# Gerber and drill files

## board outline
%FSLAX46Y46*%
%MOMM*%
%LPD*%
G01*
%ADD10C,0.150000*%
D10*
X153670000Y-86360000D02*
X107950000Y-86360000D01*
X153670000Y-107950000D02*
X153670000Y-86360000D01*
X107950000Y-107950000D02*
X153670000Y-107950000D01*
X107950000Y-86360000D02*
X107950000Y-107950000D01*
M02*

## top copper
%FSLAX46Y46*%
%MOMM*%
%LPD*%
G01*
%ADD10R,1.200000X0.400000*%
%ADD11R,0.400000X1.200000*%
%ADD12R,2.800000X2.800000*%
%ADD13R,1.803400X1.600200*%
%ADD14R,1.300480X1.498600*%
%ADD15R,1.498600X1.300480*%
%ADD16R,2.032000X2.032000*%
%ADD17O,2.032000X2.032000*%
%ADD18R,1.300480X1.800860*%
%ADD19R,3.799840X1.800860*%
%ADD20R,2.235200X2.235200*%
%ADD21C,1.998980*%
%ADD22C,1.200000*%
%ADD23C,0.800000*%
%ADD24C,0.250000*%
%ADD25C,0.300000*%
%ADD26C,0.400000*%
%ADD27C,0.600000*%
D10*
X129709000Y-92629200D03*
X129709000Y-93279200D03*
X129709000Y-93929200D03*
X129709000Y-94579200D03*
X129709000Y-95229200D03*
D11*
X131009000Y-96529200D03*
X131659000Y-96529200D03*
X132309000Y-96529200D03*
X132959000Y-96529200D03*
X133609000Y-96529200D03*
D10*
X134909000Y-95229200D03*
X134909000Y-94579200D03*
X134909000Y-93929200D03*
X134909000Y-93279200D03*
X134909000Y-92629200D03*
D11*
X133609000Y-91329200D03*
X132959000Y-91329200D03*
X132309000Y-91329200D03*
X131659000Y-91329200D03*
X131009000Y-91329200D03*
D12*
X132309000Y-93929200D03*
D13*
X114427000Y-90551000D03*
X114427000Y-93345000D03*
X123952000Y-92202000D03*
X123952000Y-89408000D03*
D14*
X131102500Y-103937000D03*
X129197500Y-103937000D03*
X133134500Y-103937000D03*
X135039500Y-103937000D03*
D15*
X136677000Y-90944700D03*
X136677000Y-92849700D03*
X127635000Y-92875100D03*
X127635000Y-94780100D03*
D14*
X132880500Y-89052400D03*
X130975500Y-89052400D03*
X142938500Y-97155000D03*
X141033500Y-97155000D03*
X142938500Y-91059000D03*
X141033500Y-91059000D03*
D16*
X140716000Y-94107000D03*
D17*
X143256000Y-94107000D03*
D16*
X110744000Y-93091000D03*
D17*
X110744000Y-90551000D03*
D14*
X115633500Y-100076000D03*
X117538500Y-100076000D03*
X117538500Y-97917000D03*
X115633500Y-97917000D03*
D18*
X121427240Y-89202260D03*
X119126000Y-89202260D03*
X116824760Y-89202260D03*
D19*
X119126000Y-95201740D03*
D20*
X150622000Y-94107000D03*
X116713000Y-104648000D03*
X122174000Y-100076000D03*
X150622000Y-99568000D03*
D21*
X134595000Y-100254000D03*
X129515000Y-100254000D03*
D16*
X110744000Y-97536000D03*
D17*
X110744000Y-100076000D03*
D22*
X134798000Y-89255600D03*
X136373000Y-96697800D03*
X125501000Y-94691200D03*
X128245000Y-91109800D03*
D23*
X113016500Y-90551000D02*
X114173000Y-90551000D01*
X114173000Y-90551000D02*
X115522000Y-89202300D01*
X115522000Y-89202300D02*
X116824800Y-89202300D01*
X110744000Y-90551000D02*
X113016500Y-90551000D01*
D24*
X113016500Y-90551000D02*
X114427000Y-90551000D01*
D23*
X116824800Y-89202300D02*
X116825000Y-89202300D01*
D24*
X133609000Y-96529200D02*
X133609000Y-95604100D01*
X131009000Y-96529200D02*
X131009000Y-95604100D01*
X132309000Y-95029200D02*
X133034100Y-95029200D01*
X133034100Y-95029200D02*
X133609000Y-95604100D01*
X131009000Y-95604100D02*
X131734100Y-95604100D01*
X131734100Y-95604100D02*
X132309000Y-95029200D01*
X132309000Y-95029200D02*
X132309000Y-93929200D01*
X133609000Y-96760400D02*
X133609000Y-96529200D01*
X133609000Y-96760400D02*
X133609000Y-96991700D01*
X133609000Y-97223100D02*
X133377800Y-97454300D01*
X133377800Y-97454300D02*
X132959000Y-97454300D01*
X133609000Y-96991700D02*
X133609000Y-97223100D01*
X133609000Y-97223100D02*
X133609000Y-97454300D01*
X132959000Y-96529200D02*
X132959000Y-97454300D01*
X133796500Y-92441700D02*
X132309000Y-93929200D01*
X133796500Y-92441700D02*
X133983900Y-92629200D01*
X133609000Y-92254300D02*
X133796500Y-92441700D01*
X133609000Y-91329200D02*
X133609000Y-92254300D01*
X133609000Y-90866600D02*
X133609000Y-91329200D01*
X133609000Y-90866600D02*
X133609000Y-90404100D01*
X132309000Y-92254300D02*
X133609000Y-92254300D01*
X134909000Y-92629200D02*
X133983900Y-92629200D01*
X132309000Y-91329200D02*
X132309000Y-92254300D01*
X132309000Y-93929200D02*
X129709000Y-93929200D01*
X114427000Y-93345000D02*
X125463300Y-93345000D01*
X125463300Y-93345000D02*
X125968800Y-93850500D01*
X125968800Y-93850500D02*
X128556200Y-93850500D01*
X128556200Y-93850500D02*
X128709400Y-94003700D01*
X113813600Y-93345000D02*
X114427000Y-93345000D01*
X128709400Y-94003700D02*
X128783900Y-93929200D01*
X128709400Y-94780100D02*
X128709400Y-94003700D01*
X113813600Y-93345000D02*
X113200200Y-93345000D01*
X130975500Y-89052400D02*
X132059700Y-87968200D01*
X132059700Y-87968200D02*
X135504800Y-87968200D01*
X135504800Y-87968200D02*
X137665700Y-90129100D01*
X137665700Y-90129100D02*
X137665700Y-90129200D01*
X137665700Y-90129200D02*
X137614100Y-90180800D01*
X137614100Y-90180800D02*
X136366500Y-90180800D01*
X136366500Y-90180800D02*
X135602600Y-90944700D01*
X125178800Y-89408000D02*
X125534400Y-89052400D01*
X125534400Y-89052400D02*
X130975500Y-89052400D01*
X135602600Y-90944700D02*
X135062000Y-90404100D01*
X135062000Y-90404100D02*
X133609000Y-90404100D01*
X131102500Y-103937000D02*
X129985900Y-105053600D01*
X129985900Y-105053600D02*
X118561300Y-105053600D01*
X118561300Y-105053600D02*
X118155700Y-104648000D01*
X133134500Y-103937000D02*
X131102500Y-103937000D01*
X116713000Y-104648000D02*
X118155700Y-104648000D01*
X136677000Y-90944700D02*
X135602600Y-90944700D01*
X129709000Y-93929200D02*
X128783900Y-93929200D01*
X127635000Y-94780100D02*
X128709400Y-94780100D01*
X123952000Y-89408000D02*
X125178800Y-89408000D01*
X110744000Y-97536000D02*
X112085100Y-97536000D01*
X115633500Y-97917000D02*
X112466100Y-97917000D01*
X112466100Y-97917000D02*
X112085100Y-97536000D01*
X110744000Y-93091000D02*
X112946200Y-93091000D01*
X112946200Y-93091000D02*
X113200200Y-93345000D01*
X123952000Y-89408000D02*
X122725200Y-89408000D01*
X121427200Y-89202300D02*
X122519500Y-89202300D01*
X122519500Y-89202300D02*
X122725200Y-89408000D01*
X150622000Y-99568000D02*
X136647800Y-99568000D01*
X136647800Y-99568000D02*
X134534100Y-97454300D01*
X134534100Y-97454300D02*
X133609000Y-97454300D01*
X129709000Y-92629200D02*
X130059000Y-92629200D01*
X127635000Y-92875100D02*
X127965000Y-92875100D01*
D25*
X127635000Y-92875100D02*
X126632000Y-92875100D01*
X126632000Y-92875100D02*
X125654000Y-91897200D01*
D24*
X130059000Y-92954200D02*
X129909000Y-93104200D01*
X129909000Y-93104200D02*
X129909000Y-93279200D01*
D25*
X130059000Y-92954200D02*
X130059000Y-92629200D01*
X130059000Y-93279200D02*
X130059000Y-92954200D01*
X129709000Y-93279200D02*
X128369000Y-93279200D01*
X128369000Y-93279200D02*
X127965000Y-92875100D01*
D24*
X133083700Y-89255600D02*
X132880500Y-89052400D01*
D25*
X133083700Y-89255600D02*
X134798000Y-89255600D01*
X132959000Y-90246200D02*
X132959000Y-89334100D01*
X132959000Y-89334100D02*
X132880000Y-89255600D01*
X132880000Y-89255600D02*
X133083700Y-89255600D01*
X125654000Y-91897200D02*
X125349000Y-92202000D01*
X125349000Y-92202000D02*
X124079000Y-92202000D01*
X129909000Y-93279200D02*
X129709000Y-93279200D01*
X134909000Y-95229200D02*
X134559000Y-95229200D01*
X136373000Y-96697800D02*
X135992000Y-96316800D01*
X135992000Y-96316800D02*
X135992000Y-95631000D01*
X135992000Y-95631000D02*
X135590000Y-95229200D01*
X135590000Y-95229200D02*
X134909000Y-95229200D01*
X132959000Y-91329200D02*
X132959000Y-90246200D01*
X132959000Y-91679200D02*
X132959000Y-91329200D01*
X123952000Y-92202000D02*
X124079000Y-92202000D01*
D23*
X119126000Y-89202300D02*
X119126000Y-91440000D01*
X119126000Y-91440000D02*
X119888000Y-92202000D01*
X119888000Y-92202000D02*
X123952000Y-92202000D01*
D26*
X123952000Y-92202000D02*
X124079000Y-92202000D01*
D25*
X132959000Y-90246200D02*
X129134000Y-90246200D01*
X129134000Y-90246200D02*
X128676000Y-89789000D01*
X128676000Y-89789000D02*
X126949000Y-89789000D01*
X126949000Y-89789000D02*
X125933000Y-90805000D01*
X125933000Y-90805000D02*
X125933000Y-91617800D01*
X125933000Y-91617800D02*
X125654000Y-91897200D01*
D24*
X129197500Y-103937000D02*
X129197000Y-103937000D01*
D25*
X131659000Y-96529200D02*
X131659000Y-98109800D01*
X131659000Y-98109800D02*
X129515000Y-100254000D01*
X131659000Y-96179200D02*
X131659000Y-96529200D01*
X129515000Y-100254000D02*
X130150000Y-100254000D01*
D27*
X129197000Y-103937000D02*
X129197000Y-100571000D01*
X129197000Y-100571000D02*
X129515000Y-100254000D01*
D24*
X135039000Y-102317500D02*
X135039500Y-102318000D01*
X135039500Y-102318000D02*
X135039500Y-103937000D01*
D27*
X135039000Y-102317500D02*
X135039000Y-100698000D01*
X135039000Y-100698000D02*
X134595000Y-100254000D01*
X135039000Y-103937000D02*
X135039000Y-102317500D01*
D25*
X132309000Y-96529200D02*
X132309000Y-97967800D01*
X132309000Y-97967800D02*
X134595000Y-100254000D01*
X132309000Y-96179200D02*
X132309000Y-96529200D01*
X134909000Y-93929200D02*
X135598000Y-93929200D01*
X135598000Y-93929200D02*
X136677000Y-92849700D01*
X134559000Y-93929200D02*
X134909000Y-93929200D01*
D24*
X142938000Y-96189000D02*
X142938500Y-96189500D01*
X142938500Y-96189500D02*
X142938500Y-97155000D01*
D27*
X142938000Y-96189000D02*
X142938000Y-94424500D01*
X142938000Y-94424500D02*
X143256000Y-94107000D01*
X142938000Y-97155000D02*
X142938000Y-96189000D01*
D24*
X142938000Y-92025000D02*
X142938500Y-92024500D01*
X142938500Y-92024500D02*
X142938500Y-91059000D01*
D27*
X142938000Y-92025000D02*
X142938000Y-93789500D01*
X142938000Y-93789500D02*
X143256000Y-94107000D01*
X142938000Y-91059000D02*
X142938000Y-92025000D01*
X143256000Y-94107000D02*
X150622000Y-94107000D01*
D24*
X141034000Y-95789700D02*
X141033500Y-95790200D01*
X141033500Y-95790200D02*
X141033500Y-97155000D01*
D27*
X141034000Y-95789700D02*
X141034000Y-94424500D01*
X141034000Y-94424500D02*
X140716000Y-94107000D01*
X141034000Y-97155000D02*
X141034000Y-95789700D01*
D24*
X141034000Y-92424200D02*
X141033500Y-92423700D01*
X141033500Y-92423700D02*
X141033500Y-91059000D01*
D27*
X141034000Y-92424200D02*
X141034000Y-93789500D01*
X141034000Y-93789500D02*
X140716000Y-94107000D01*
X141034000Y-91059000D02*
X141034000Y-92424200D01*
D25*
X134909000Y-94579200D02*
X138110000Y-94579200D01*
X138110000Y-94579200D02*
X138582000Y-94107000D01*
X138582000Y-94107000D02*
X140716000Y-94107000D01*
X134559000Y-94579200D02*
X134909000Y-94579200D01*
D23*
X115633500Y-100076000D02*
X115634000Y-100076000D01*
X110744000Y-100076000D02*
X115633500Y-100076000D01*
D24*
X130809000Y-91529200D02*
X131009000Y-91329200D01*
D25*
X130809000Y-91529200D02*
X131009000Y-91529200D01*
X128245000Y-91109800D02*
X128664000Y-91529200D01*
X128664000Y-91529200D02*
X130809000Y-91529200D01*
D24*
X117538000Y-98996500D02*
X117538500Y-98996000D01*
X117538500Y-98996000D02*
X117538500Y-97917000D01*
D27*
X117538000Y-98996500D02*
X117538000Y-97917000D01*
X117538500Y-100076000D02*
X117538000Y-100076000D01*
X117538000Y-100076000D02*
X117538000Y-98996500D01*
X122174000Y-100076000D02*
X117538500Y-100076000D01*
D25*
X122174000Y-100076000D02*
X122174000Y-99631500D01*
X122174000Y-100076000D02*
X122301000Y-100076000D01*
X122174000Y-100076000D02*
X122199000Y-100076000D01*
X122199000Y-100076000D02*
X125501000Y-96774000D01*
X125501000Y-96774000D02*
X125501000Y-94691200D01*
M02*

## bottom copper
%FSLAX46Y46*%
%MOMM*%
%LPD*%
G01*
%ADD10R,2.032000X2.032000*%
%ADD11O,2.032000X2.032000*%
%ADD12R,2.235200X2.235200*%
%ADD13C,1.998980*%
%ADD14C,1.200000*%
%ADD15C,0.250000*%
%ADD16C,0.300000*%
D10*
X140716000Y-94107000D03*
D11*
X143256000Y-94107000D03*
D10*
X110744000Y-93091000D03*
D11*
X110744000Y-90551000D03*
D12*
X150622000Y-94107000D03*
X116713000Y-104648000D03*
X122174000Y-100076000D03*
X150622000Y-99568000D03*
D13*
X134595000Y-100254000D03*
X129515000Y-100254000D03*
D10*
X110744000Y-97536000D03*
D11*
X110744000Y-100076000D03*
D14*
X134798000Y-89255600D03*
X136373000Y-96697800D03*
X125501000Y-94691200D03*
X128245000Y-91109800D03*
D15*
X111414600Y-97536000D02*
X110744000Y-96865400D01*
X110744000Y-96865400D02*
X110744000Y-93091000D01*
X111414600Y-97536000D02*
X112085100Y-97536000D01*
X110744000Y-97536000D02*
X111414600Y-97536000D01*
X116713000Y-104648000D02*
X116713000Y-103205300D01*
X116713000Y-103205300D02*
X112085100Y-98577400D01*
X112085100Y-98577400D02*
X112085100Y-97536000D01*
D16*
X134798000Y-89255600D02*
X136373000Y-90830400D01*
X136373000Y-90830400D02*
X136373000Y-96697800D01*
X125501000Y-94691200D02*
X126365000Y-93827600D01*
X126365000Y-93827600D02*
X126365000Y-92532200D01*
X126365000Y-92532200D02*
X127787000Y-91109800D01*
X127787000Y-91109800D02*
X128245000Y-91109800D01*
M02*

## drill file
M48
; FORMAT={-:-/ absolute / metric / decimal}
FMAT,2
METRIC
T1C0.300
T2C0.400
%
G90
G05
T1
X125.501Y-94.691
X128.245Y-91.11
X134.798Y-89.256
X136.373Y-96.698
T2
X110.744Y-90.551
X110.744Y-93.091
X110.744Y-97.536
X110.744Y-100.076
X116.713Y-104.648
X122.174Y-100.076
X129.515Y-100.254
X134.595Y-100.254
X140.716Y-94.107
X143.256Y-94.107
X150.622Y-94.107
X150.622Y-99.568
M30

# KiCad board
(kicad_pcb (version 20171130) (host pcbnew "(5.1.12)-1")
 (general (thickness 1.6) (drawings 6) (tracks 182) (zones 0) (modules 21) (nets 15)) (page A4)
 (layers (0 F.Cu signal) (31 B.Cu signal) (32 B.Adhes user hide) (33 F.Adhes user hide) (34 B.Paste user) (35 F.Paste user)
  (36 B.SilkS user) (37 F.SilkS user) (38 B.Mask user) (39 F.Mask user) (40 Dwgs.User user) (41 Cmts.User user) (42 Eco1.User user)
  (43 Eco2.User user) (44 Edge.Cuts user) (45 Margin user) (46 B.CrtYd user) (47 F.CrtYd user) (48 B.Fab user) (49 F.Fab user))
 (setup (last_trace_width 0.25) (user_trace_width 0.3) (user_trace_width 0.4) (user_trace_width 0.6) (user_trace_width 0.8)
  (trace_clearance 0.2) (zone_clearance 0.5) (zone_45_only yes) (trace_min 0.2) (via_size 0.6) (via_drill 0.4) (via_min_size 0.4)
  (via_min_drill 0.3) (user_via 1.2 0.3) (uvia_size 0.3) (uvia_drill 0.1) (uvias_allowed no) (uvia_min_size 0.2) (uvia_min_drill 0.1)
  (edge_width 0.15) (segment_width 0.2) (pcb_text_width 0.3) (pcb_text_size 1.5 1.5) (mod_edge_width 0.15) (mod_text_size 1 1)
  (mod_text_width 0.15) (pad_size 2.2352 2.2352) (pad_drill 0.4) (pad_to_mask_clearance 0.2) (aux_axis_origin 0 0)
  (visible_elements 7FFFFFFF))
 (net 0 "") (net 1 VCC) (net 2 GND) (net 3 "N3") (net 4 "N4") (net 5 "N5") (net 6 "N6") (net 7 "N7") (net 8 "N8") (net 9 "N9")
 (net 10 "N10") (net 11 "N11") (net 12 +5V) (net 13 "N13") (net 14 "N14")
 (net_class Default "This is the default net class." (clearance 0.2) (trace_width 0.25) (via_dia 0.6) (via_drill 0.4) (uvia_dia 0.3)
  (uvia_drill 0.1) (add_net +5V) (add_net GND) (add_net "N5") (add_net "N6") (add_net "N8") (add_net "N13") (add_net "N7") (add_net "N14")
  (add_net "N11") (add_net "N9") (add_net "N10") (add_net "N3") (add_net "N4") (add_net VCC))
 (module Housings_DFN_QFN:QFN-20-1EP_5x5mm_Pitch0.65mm (layer F.Cu) (at 132.309 93.9292)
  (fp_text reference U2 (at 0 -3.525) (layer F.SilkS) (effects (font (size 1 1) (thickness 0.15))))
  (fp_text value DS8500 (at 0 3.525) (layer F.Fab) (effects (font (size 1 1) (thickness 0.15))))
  (pad 1 smd rect (at -2.6 -1.3) (size 1.2 0.4) (layers F.Cu F.Paste F.Mask) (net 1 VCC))
  (pad 2 smd rect (at -2.6 -0.65) (size 1.2 0.4) (layers F.Cu F.Paste F.Mask) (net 1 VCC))
  (pad 3 smd rect (at -2.6 0) (size 1.2 0.4) (layers F.Cu F.Paste F.Mask) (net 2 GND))
  (pad 4 smd rect (at -2.6 0.65) (size 1.2 0.4) (layers F.Cu F.Paste F.Mask) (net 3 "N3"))
  (pad 5 smd rect (at -2.6 1.3) (size 1.2 0.4) (layers F.Cu F.Paste F.Mask) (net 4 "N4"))
  (pad 6 smd rect (at -1.3 2.6 90) (size 1.2 0.4) (layers F.Cu F.Paste F.Mask) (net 2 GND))
  (pad 7 smd rect (at -0.65 2.6 90) (size 1.2 0.4) (layers F.Cu F.Paste F.Mask) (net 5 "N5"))
  (pad 8 smd rect (at 0 2.6 90) (size 1.2 0.4) (layers F.Cu F.Paste F.Mask) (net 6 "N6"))
  (pad 9 smd rect (at 0.65 2.6 90) (size 1.2 0.4) (layers F.Cu F.Paste F.Mask) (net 2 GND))
  (pad 10 smd rect (at 1.3 2.6 90) (size 1.2 0.4) (layers F.Cu F.Paste F.Mask) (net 2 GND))
  (pad 11 smd rect (at 2.6 1.3) (size 1.2 0.4) (layers F.Cu F.Paste F.Mask) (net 1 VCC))
  (pad 12 smd rect (at 2.6 0.65) (size 1.2 0.4) (layers F.Cu F.Paste F.Mask) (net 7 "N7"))
  (pad 13 smd rect (at 2.6 0) (size 1.2 0.4) (layers F.Cu F.Paste F.Mask) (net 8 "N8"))
  (pad 14 smd rect (at 2.6 -0.65) (size 1.2 0.4) (layers F.Cu F.Paste F.Mask) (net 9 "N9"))
  (pad 15 smd rect (at 2.6 -1.3) (size 1.2 0.4) (layers F.Cu F.Paste F.Mask) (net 2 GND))
  (pad 16 smd rect (at 1.3 -2.6 90) (size 1.2 0.4) (layers F.Cu F.Paste F.Mask) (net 2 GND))
  (pad 17 smd rect (at 0.65 -2.6 90) (size 1.2 0.4) (layers F.Cu F.Paste F.Mask) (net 1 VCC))
  (pad 18 smd rect (at 0 -2.6 90) (size 1.2 0.4) (layers F.Cu F.Paste F.Mask) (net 2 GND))
  (pad 19 smd rect (at -0.65 -2.6 90) (size 1.2 0.4) (layers F.Cu F.Paste F.Mask) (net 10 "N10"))
  (pad 20 smd rect (at -1.3 -2.6 90) (size 1.2 0.4) (layers F.Cu F.Paste F.Mask) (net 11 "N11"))
  (pad 21 smd rect (at 0 0) (size 2.8 2.8) (layers F.Cu F.Paste F.Mask) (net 2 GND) (solder_paste_margin_ratio -0.2)))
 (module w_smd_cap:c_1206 (layer F.Cu) (at 114.427 91.948 90)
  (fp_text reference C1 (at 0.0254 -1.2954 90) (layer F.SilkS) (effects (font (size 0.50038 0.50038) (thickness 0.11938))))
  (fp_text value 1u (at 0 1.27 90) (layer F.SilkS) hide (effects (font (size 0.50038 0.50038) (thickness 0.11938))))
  (pad 1 smd rect (at 1.397 0 90) (size 1.6002 1.8034) (layers F.Cu F.Paste F.Mask) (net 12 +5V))
  (pad 2 smd rect (at -1.397 0 90) (size 1.6002 1.8034) (layers F.Cu F.Paste F.Mask) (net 2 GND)))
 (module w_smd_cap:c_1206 (layer F.Cu) (at 123.952 90.805 270)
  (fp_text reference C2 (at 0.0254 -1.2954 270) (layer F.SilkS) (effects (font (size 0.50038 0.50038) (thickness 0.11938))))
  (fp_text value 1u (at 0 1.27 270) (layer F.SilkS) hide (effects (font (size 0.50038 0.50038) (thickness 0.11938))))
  (pad 1 smd rect (at 1.397 0 270) (size 1.6002 1.8034) (layers F.Cu F.Paste F.Mask) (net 1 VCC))
  (pad 2 smd rect (at -1.397 0 270) (size 1.6002 1.8034) (layers F.Cu F.Paste F.Mask) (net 2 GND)))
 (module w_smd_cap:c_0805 (layer F.Cu) (at 130.15 103.937)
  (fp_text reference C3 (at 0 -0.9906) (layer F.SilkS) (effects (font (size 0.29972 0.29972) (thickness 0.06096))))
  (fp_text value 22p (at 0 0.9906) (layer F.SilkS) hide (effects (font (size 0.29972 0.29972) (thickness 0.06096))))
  (pad 1 smd rect (at 0.9525 0) (size 1.30048 1.4986) (layers F.Cu F.Paste F.Mask) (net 2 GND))
  (pad 2 smd rect (at -0.9525 0) (size 1.30048 1.4986) (layers F.Cu F.Paste F.Mask) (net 5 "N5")))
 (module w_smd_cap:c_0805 (layer F.Cu) (at 134.087 103.937 180)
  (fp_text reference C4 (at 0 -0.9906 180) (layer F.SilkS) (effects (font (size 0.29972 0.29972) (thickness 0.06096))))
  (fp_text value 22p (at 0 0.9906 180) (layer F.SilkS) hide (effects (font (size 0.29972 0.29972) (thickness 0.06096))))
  (pad 1 smd rect (at 0.9525 0 180) (size 1.30048 1.4986) (layers F.Cu F.Paste F.Mask) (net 2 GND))
  (pad 2 smd rect (at -0.9525 0 180) (size 1.30048 1.4986) (layers F.Cu F.Paste F.Mask) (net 6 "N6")))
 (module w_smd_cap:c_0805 (layer F.Cu) (at 136.677 91.8972 90)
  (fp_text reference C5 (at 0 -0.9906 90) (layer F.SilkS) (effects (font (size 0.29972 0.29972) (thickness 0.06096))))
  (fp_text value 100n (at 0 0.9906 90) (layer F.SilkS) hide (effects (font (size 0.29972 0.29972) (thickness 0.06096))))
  (pad 1 smd rect (at 0.9525 0 90) (size 1.30048 1.4986) (layers F.Cu F.Paste F.Mask) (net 2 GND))
  (pad 2 smd rect (at -0.9525 0 90) (size 1.30048 1.4986) (layers F.Cu F.Paste F.Mask) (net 8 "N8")))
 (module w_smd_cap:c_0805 (layer F.Cu) (at 127.635 93.8276 90)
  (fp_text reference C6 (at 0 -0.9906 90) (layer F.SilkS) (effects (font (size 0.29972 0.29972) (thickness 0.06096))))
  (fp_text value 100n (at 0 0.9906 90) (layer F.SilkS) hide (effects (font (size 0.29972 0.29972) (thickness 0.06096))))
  (pad 1 smd rect (at 0.9525 0 90) (size 1.30048 1.4986) (layers F.Cu F.Paste F.Mask) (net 1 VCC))
  (pad 2 smd rect (at -0.9525 0 90) (size 1.30048 1.4986) (layers F.Cu F.Paste F.Mask) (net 2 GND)))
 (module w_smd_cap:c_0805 (layer F.Cu) (at 131.928 89.0524)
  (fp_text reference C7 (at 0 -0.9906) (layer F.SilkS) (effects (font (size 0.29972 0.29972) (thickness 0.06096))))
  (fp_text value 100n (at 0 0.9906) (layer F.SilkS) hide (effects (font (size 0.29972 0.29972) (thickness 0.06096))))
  (pad 1 smd rect (at 0.9525 0) (size 1.30048 1.4986) (layers F.Cu F.Paste F.Mask) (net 1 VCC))
  (pad 2 smd rect (at -0.9525 0) (size 1.30048 1.4986) (layers F.Cu F.Paste F.Mask) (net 2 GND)))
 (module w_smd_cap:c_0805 (layer F.Cu) (at 141.986 97.155)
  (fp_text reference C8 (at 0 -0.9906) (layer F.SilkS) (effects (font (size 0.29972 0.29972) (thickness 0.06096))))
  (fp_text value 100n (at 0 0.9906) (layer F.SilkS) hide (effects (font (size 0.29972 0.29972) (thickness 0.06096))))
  (pad 1 smd rect (at 0.9525 0) (size 1.30048 1.4986) (layers F.Cu F.Paste F.Mask) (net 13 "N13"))
  (pad 2 smd rect (at -0.9525 0) (size 1.30048 1.4986) (layers F.Cu F.Paste F.Mask) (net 7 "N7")))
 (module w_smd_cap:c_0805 (layer F.Cu) (at 141.986 91.059)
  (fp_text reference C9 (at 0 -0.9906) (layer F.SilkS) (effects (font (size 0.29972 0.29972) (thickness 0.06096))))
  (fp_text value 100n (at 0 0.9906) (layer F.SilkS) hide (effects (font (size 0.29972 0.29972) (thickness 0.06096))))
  (pad 1 smd rect (at 0.9525 0) (size 1.30048 1.4986) (layers F.Cu F.Paste F.Mask) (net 13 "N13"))
  (pad 2 smd rect (at -0.9525 0) (size 1.30048 1.4986) (layers F.Cu F.Paste F.Mask) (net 7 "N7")))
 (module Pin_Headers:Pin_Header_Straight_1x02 (layer F.Cu) (at 140.716 94.107 90)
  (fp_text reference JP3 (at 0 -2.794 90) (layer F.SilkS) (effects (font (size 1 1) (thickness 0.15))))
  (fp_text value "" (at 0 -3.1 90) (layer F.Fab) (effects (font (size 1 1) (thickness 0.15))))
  (pad 1 thru_hole rect (at 0 0 90) (size 2.032 2.032) (drill 0.4) (layers *.Cu *.Mask F.SilkS) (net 7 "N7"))
  (pad 2 thru_hole oval (at 0 2.54 90) (size 2.032 2.032) (drill 0.4) (layers *.Cu *.Mask F.SilkS) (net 13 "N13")))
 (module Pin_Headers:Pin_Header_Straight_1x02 (layer F.Cu) (at 110.744 93.091 180)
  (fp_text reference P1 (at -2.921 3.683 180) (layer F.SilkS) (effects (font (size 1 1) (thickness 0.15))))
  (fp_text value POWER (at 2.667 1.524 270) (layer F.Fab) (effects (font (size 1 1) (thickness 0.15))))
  (pad 1 thru_hole rect (at 0 0 180) (size 2.032 2.032) (drill 0.4) (layers *.Cu *.Mask F.SilkS) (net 2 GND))
  (pad 2 thru_hole oval (at 0 2.54 180) (size 2.032 2.032) (drill 0.4) (layers *.Cu *.Mask F.SilkS) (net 12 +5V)))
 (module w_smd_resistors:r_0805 (layer F.Cu) (at 116.586 100.076 180)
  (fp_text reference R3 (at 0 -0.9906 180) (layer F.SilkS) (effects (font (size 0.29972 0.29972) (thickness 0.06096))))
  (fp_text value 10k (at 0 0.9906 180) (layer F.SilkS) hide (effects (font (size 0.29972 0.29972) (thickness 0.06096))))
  (pad 1 smd rect (at 0.9525 0 180) (size 1.30048 1.4986) (layers F.Cu F.Paste F.Mask) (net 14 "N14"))
  (pad 2 smd rect (at -0.9525 0 180) (size 1.30048 1.4986) (layers F.Cu F.Paste F.Mask) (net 11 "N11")))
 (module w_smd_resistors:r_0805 (layer F.Cu) (at 116.586 97.917)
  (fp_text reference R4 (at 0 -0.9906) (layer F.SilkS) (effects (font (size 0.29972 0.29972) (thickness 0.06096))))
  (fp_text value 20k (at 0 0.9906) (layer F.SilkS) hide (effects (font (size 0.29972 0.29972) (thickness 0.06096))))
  (pad 1 smd rect (at 0.9525 0) (size 1.30048 1.4986) (layers F.Cu F.Paste F.Mask) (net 11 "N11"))
  (pad 2 smd rect (at -0.9525 0) (size 1.30048 1.4986) (layers F.Cu F.Paste F.Mask) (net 2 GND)))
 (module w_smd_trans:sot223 (layer F.Cu) (at 119.126 92.202 180)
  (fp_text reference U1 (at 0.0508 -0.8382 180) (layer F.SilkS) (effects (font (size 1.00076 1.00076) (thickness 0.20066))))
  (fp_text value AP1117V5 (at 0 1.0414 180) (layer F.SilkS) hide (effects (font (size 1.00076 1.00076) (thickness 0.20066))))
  (pad 1 smd rect (at -2.30124 2.99974 180) (size 1.30048 1.80086) (layers F.Cu F.Paste F.Mask) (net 2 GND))
  (pad 2 smd rect (at 0 2.99974 180) (size 1.30048 1.80086) (layers F.Cu F.Paste F.Mask) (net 1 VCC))
  (pad 3 smd rect (at 2.30124 2.99974 180) (size 1.30048 1.80086) (layers F.Cu F.Paste F.Mask) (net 12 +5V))
  (pad 4 smd rect (at 0 -2.99974 180) (size 3.79984 1.80086) (layers F.Cu F.Paste F.Mask)))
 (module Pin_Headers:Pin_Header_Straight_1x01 (layer F.Cu) (at 150.622 94.107)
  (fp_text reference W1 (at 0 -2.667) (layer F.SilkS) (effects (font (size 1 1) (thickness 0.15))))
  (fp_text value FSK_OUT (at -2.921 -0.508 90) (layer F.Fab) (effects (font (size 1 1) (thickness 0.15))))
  (pad 1 thru_hole rect (at 0 0) (size 2.2352 2.2352) (drill 0.4) (layers *.Cu *.Mask F.SilkS) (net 13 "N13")))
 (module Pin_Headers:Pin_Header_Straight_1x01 (layer F.Cu) (at 116.713 104.648)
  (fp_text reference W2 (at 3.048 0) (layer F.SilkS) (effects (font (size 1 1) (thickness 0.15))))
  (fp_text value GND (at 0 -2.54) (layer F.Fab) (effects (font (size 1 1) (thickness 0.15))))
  (pad 1 thru_hole rect (at 0 0) (size 2.2352 2.2352) (drill 0.4) (layers *.Cu *.Mask F.SilkS) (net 2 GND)))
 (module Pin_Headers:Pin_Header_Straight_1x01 (layer F.Cu) (at 122.174 100.076)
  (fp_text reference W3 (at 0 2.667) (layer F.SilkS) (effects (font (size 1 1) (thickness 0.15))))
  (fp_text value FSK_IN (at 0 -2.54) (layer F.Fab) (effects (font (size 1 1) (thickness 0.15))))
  (pad 1 thru_hole rect (at 0 0) (size 2.2352 2.2352) (drill 0.4) (layers *.Cu *.Mask F.SilkS) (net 11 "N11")))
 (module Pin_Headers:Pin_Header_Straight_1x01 (layer F.Cu) (at 150.622 99.568)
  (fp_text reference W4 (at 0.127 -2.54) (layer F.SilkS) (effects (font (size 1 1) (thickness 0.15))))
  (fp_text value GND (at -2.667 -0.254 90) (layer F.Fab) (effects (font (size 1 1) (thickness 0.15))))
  (pad 1 thru_hole rect (at 0 0) (size 2.2352 2.2352) (drill 0.4) (layers *.Cu *.Mask F.SilkS) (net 2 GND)))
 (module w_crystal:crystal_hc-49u (layer F.Cu) (at 132.055 100.254 180) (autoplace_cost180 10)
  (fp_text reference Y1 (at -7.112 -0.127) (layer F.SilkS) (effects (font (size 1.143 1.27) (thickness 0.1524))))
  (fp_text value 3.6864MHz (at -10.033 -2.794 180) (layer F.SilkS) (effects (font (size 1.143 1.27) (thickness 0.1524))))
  (pad 1 thru_hole circle (at -2.54 0 180) (size 1.99898 1.99898) (drill 0.4) (layers *.Cu *.Mask F.SilkS) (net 6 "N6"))
  (pad 2 thru_hole circle (at 2.54 0 180) (size 1.99898 1.99898) (drill 0.4) (layers *.Cu *.Mask F.SilkS) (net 5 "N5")))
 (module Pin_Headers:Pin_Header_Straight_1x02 (layer F.Cu) (at 110.744 97.536)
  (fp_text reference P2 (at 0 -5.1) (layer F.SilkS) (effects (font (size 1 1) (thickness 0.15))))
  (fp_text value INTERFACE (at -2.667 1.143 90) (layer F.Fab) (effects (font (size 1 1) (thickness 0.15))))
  (pad 1 thru_hole rect (at 0 0) (size 2.032 2.032) (drill 0.4) (layers *.Cu *.Mask F.SilkS) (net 2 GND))
  (pad 2 thru_hole oval (at 0 2.54) (size 2.032 2.032) (drill 0.4) (layers *.Cu *.Mask F.SilkS) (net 14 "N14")))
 (gr_line (start 153.67 86.36) (end 107.95 86.36) (angle 90) (layer Edge.Cuts) (width 0.15))
 (gr_line (start 153.67 107.95) (end 153.67 86.36) (angle 90) (layer Edge.Cuts) (width 0.15))
 (gr_line (start 107.95 107.95) (end 153.67 107.95) (angle 90) (layer Edge.Cuts) (width 0.15))
 (gr_line (start 107.95 86.36) (end 107.95 107.95) (angle 90) (layer Edge.Cuts) (width 0.15))
 (segment (start 113.0165 90.551) (end 114.173 90.551) (width 0.8) (layer F.Cu) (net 12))
 (segment (start 114.173 90.551) (end 115.522 89.2023) (width 0.8) (layer F.Cu) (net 12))
 (segment (start 115.522 89.2023) (end 116.8248 89.2023) (width 0.8) (layer F.Cu) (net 12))
 (segment (start 110.744 90.551) (end 113.0165 90.551) (width 0.8) (layer F.Cu) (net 12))
 (segment (start 113.0165 90.551) (end 114.427 90.551) (width 0.25) (layer F.Cu) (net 12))
 (segment (start 116.8248 89.2023) (end 116.825 89.2023) (width 0.8) (layer F.Cu) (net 12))
 (segment (start 133.609 96.5292) (end 133.609 95.6041) (width 0.25) (layer F.Cu) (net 2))
 (segment (start 131.009 96.5292) (end 131.009 95.6041) (width 0.25) (layer F.Cu) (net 2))
 (segment (start 132.309 95.0292) (end 133.0341 95.0292) (width 0.25) (layer F.Cu) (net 2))
 (segment (start 133.0341 95.0292) (end 133.609 95.6041) (width 0.25) (layer F.Cu) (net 2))
 (segment (start 131.009 95.6041) (end 131.7341 95.6041) (width 0.25) (layer F.Cu) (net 2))
 (segment (start 131.7341 95.6041) (end 132.309 95.0292) (width 0.25) (layer F.Cu) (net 2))
 (segment (start 132.309 95.0292) (end 132.309 93.9292) (width 0.25) (layer F.Cu) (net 2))
 (segment (start 133.609 96.7604) (end 133.609 96.5292) (width 0.25) (layer F.Cu) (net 2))
 (segment (start 133.609 96.7604) (end 133.609 96.9917) (width 0.25) (layer F.Cu) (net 2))
 (segment (start 133.609 97.2231) (end 133.3778 97.4543) (width 0.25) (layer F.Cu) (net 2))
 (segment (start 133.3778 97.4543) (end 132.959 97.4543) (width 0.25) (layer F.Cu) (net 2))
 (segment (start 133.609 96.9917) (end 133.609 97.2231) (width 0.25) (layer F.Cu) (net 2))
 (segment (start 133.609 97.2231) (end 133.609 97.4543) (width 0.25) (layer F.Cu) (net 2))
 (segment (start 132.959 96.5292) (end 132.959 97.4543) (width 0.25) (layer F.Cu) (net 2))
 (segment (start 133.7965 92.4417) (end 132.309 93.9292) (width 0.25) (layer F.Cu) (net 2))
 (segment (start 133.7965 92.4417) (end 133.9839 92.6292) (width 0.25) (layer F.Cu) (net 2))
 (segment (start 133.609 92.2543) (end 133.7965 92.4417) (width 0.25) (layer F.Cu) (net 2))
 (segment (start 133.609 91.3292) (end 133.609 92.2543) (width 0.25) (layer F.Cu) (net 2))
 (segment (start 133.609 90.8666) (end 133.609 91.3292) (width 0.25) (layer F.Cu) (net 2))
 (segment (start 133.609 90.8666) (end 133.609 90.4041) (width 0.25) (layer F.Cu) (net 2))
 (segment (start 132.309 92.2543) (end 133.609 92.2543) (width 0.25) (layer F.Cu) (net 2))
 (segment (start 134.909 92.6292) (end 133.9839 92.6292) (width 0.25) (layer F.Cu) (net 2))
 (segment (start 132.309 91.3292) (end 132.309 92.2543) (width 0.25) (layer F.Cu) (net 2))
 (segment (start 132.309 93.9292) (end 129.709 93.9292) (width 0.25) (layer F.Cu) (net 2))
 (segment (start 114.427 93.345) (end 125.4633 93.345) (width 0.25) (layer F.Cu) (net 2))
 (segment (start 125.4633 93.345) (end 125.9688 93.8505) (width 0.25) (layer F.Cu) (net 2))
 (segment (start 125.9688 93.8505) (end 128.5562 93.8505) (width 0.25) (layer F.Cu) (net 2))
 (segment (start 128.5562 93.8505) (end 128.7094 94.0037) (width 0.25) (layer F.Cu) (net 2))
 (segment (start 113.8136 93.345) (end 114.427 93.345) (width 0.25) (layer F.Cu) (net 2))
 (segment (start 128.7094 94.0037) (end 128.7839 93.9292) (width 0.25) (layer F.Cu) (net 2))
 (segment (start 128.7094 94.7801) (end 128.7094 94.0037) (width 0.25) (layer F.Cu) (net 2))
 (segment (start 113.8136 93.345) (end 113.2002 93.345) (width 0.25) (layer F.Cu) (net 2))
 (segment (start 130.9755 89.0524) (end 132.0597 87.9682) (width 0.25) (layer F.Cu) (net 2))
 (segment (start 132.0597 87.9682) (end 135.5048 87.9682) (width 0.25) (layer F.Cu) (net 2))
 (segment (start 135.5048 87.9682) (end 137.6657 90.1291) (width 0.25) (layer F.Cu) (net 2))
 (segment (start 137.6657 90.1291) (end 137.6657 90.1292) (width 0.25) (layer F.Cu) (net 2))
 (segment (start 137.6657 90.1292) (end 137.6141 90.1808) (width 0.25) (layer F.Cu) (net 2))
 (segment (start 137.6141 90.1808) (end 136.3665 90.1808) (width 0.25) (layer F.Cu) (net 2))
 (segment (start 136.3665 90.1808) (end 135.6026 90.9447) (width 0.25) (layer F.Cu) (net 2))
 (segment (start 125.1788 89.408) (end 125.5344 89.0524) (width 0.25) (layer F.Cu) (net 2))
 (segment (start 125.5344 89.0524) (end 130.9755 89.0524) (width 0.25) (layer F.Cu) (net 2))
 (segment (start 135.6026 90.9447) (end 135.062 90.4041) (width 0.25) (layer F.Cu) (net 2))
 (segment (start 135.062 90.4041) (end 133.609 90.4041) (width 0.25) (layer F.Cu) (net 2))
 (segment (start 131.1025 103.937) (end 129.9859 105.0536) (width 0.25) (layer F.Cu) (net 2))
 (segment (start 129.9859 105.0536) (end 118.5613 105.0536) (width 0.25) (layer F.Cu) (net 2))
 (segment (start 118.5613 105.0536) (end 118.1557 104.648) (width 0.25) (layer F.Cu) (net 2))
 (segment (start 133.1345 103.937) (end 131.1025 103.937) (width 0.25) (layer F.Cu) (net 2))
 (segment (start 116.713 104.648) (end 118.1557 104.648) (width 0.25) (layer F.Cu) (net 2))
 (segment (start 136.677 90.9447) (end 135.6026 90.9447) (width 0.25) (layer F.Cu) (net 2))
 (segment (start 129.709 93.9292) (end 128.7839 93.9292) (width 0.25) (layer F.Cu) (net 2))
 (segment (start 127.635 94.7801) (end 128.7094 94.7801) (width 0.25) (layer F.Cu) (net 2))
 (segment (start 123.952 89.408) (end 125.1788 89.408) (width 0.25) (layer F.Cu) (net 2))
 (segment (start 110.744 97.536) (end 112.0851 97.536) (width 0.25) (layer F.Cu) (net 2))
 (segment (start 115.6335 97.917) (end 112.4661 97.917) (width 0.25) (layer F.Cu) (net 2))
 (segment (start 112.4661 97.917) (end 112.0851 97.536) (width 0.25) (layer F.Cu) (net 2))
 (segment (start 110.744 93.091) (end 112.9462 93.091) (width 0.25) (layer F.Cu) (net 2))
 (segment (start 112.9462 93.091) (end 113.2002 93.345) (width 0.25) (layer F.Cu) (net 2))
 (segment (start 111.4146 97.536) (end 110.744 96.8654) (width 0.25) (layer B.Cu) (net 2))
 (segment (start 110.744 96.8654) (end 110.744 93.091) (width 0.25) (layer B.Cu) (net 2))
 (segment (start 111.4146 97.536) (end 112.0851 97.536) (width 0.25) (layer B.Cu) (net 2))
 (segment (start 110.744 97.536) (end 111.4146 97.536) (width 0.25) (layer B.Cu) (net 2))
 (segment (start 123.952 89.408) (end 122.7252 89.408) (width 0.25) (layer F.Cu) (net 2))
 (segment (start 121.4272 89.2023) (end 122.5195 89.2023) (width 0.25) (layer F.Cu) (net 2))
 (segment (start 122.5195 89.2023) (end 122.7252 89.408) (width 0.25) (layer F.Cu) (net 2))
 (segment (start 116.713 104.648) (end 116.713 103.2053) (width 0.25) (layer B.Cu) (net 2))
 (segment (start 116.713 103.2053) (end 112.0851 98.5774) (width 0.25) (layer B.Cu) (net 2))
 (segment (start 112.0851 98.5774) (end 112.0851 97.536) (width 0.25) (layer B.Cu) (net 2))
 (segment (start 150.622 99.568) (end 136.6478 99.568) (width 0.25) (layer F.Cu) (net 2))
 (segment (start 136.6478 99.568) (end 134.5341 97.4543) (width 0.25) (layer F.Cu) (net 2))
 (segment (start 134.5341 97.4543) (end 133.609 97.4543) (width 0.25) (layer F.Cu) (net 2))
 (segment (start 129.709 92.6292) (end 130.059 92.6292) (width 0.25) (layer F.Cu) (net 1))
 (segment (start 127.635 92.8751) (end 127.965 92.8751) (width 0.25) (layer F.Cu) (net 1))
 (segment (start 127.635 92.8751) (end 126.632 92.8751) (width 0.3) (layer F.Cu) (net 1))
 (segment (start 126.632 92.8751) (end 125.654 91.8972) (width 0.3) (layer F.Cu) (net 1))
 (segment (start 130.059 92.9542) (end 129.909 93.1042) (width 0.25) (layer F.Cu) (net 1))
 (segment (start 129.909 93.1042) (end 129.909 93.2792) (width 0.25) (layer F.Cu) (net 1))
 (segment (start 130.059 92.9542) (end 130.059 92.6292) (width 0.3) (layer F.Cu) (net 1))
 (segment (start 130.059 93.2792) (end 130.059 92.9542) (width 0.3) (layer F.Cu) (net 1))
 (segment (start 129.709 93.2792) (end 128.369 93.2792) (width 0.3) (layer F.Cu) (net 1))
 (segment (start 128.369 93.2792) (end 127.965 92.8751) (width 0.3) (layer F.Cu) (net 1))
 (segment (start 133.0837 89.2556) (end 132.8805 89.0524) (width 0.25) (layer F.Cu) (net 1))
 (segment (start 133.0837 89.2556) (end 134.798 89.2556) (width 0.3) (layer F.Cu) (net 1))
 (segment (start 132.959 90.2462) (end 132.959 89.3341) (width 0.3) (layer F.Cu) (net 1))
 (segment (start 132.959 89.3341) (end 132.88 89.2556) (width 0.3) (layer F.Cu) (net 1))
 (segment (start 132.88 89.2556) (end 133.0837 89.2556) (width 0.3) (layer F.Cu) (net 1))
 (segment (start 125.654 91.8972) (end 125.349 92.202) (width 0.3) (layer F.Cu) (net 1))
 (segment (start 125.349 92.202) (end 124.079 92.202) (width 0.3) (layer F.Cu) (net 1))
 (segment (start 129.909 93.2792) (end 129.709 93.2792) (width 0.3) (layer F.Cu) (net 1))
 (segment (start 134.909 95.2292) (end 134.559 95.2292) (width 0.3) (layer F.Cu) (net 1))
 (segment (start 136.373 96.6978) (end 135.992 96.3168) (width 0.3) (layer F.Cu) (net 1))
 (segment (start 135.992 96.3168) (end 135.992 95.631) (width 0.3) (layer F.Cu) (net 1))
 (segment (start 135.992 95.631) (end 135.59 95.2292) (width 0.3) (layer F.Cu) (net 1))
 (segment (start 135.59 95.2292) (end 134.909 95.2292) (width 0.3) (layer F.Cu) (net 1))
 (segment (start 132.959 91.3292) (end 132.959 90.2462) (width 0.3) (layer F.Cu) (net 1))
 (segment (start 132.959 91.6792) (end 132.959 91.3292) (width 0.3) (layer F.Cu) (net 1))
 (segment (start 123.952 92.202) (end 124.079 92.202) (width 0.3) (layer F.Cu) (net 1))
 (segment (start 119.126 89.2023) (end 119.126 91.44) (width 0.8) (layer F.Cu) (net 1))
 (segment (start 119.126 91.44) (end 119.888 92.202) (width 0.8) (layer F.Cu) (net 1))
 (segment (start 119.888 92.202) (end 123.952 92.202) (width 0.8) (layer F.Cu) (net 1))
 (segment (start 123.952 92.202) (end 124.079 92.202) (width 0.4) (layer F.Cu) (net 1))
 (segment (start 134.798 89.2556) (end 136.373 90.8304) (width 0.3) (layer B.Cu) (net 1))
 (segment (start 136.373 90.8304) (end 136.373 96.6978) (width 0.3) (layer B.Cu) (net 1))
 (segment (start 132.959 90.2462) (end 129.134 90.2462) (width 0.3) (layer F.Cu) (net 1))
 (segment (start 129.134 90.2462) (end 128.676 89.789) (width 0.3) (layer F.Cu) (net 1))
 (segment (start 128.676 89.789) (end 126.949 89.789) (width 0.3) (layer F.Cu) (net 1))
 (segment (start 126.949 89.789) (end 125.933 90.805) (width 0.3) (layer F.Cu) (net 1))
 (segment (start 125.933 90.805) (end 125.933 91.6178) (width 0.3) (layer F.Cu) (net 1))
 (segment (start 125.933 91.6178) (end 125.654 91.8972) (width 0.3) (layer F.Cu) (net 1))
 (via (at 134.798 89.2556) (size 1.2) (drill 0.3) (layers F.Cu B.Cu) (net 1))
 (via (at 136.373 96.6978) (size 1.2) (drill 0.3) (layers F.Cu B.Cu) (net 1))
 (segment (start 129.1975 103.937) (end 129.197 103.937) (width 0.25) (layer F.Cu) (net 5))
 (segment (start 131.659 96.5292) (end 131.659 98.1098) (width 0.3) (layer F.Cu) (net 5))
 (segment (start 131.659 98.1098) (end 129.515 100.254) (width 0.3) (layer F.Cu) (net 5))
 (segment (start 131.659 96.1792) (end 131.659 96.5292) (width 0.3) (layer F.Cu) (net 5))
 (segment (start 129.515 100.254) (end 130.15 100.254) (width 0.3) (layer F.Cu) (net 5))
 (segment (start 129.197 103.937) (end 129.197 100.571) (width 0.6) (layer F.Cu) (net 5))
 (segment (start 129.197 100.571) (end 129.515 100.254) (width 0.6) (layer F.Cu) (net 5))
 (segment (start 135.039 102.3175) (end 135.0395 102.318) (width 0.25) (layer F.Cu) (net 6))
 (segment (start 135.0395 102.318) (end 135.0395 103.937) (width 0.25) (layer F.Cu) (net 6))
 (segment (start 135.039 102.3175) (end 135.039 100.698) (width 0.6) (layer F.Cu) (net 6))
 (segment (start 135.039 100.698) (end 134.595 100.254) (width 0.6) (layer F.Cu) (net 6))
 (segment (start 135.039 103.937) (end 135.039 102.3175) (width 0.6) (layer F.Cu) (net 6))
 (segment (start 132.309 96.5292) (end 132.309 97.9678) (width 0.3) (layer F.Cu) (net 6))
 (segment (start 132.309 97.9678) (end 134.595 100.254) (width 0.3) (layer F.Cu) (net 6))
 (segment (start 132.309 96.1792) (end 132.309 96.5292) (width 0.3) (layer F.Cu) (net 6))
 (segment (start 134.909 93.9292) (end 135.598 93.9292) (width 0.3) (layer F.Cu) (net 8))
 (segment (start 135.598 93.9292) (end 136.677 92.8497) (width 0.3) (layer F.Cu) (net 8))
 (segment (start 134.559 93.9292) (end 134.909 93.9292) (width 0.3) (layer F.Cu) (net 8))
 (segment (start 142.938 96.189) (end 142.9385 96.1895) (width 0.25) (layer F.Cu) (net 13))
 (segment (start 142.9385 96.1895) (end 142.9385 97.155) (width 0.25) (layer F.Cu) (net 13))
 (segment (start 142.938 96.189) (end 142.938 94.4245) (width 0.6) (layer F.Cu) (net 13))
 (segment (start 142.938 94.4245) (end 143.256 94.107) (width 0.6) (layer F.Cu) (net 13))
 (segment (start 142.938 97.155) (end 142.938 96.189) (width 0.6) (layer F.Cu) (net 13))
 (segment (start 142.938 92.025) (end 142.9385 92.0245) (width 0.25) (layer F.Cu) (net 13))
 (segment (start 142.9385 92.0245) (end 142.9385 91.059) (width 0.25) (layer F.Cu) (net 13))
 (segment (start 142.938 92.025) (end 142.938 93.7895) (width 0.6) (layer F.Cu) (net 13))
 (segment (start 142.938 93.7895) (end 143.256 94.107) (width 0.6) (layer F.Cu) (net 13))
 (segment (start 142.938 91.059) (end 142.938 92.025) (width 0.6) (layer F.Cu) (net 13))
 (segment (start 143.256 94.107) (end 150.622 94.107) (width 0.6) (layer F.Cu) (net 13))
 (segment (start 141.034 95.7897) (end 141.0335 95.7902) (width 0.25) (layer F.Cu) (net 7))
 (segment (start 141.0335 95.7902) (end 141.0335 97.155) (width 0.25) (layer F.Cu) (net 7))
 (segment (start 141.034 95.7897) (end 141.034 94.4245) (width 0.6) (layer F.Cu) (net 7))
 (segment (start 141.034 94.4245) (end 140.716 94.107) (width 0.6) (layer F.Cu) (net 7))
 (segment (start 141.034 97.155) (end 141.034 95.7897) (width 0.6) (layer F.Cu) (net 7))
 (segment (start 141.034 92.4242) (end 141.0335 92.4237) (width 0.25) (layer F.Cu) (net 7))
 (segment (start 141.0335 92.4237) (end 141.0335 91.059) (width 0.25) (layer F.Cu) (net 7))
 (segment (start 141.034 92.4242) (end 141.034 93.7895) (width 0.6) (layer F.Cu) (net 7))
 (segment (start 141.034 93.7895) (end 140.716 94.107) (width 0.6) (layer F.Cu) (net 7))
 (segment (start 141.034 91.059) (end 141.034 92.4242) (width 0.6) (layer F.Cu) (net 7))
 (segment (start 134.909 94.5792) (end 138.11 94.5792) (width 0.3) (layer F.Cu) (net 7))
 (segment (start 138.11 94.5792) (end 138.582 94.107) (width 0.3) (layer F.Cu) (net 7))
 (segment (start 138.582 94.107) (end 140.716 94.107) (width 0.3) (layer F.Cu) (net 7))
 (segment (start 134.559 94.5792) (end 134.909 94.5792) (width 0.3) (layer F.Cu) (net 7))
 (segment (start 115.6335 100.076) (end 115.634 100.076) (width 0.8) (layer F.Cu) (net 14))
 (segment (start 110.744 100.076) (end 115.6335 100.076) (width 0.8) (layer F.Cu) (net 14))
 (segment (start 130.809 91.5292) (end 131.009 91.3292) (width 0.25) (layer F.Cu) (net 11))
 (segment (start 130.809 91.5292) (end 131.009 91.5292) (width 0.3) (layer F.Cu) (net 11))
 (segment (start 128.245 91.1098) (end 128.664 91.5292) (width 0.3) (layer F.Cu) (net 11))
 (segment (start 128.664 91.5292) (end 130.809 91.5292) (width 0.3) (layer F.Cu) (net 11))
 (segment (start 117.538 98.9965) (end 117.5385 98.996) (width 0.25) (layer F.Cu) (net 11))
 (segment (start 117.5385 98.996) (end 117.5385 97.917) (width 0.25) (layer F.Cu) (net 11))
 (segment (start 117.538 98.9965) (end 117.538 97.917) (width 0.6) (layer F.Cu) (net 11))
 (segment (start 117.5385 100.076) (end 117.538 100.076) (width 0.6) (layer F.Cu) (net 11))
 (segment (start 117.538 100.076) (end 117.538 98.9965) (width 0.6) (layer F.Cu) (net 11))
 (segment (start 122.174 100.076) (end 117.5385 100.076) (width 0.6) (layer F.Cu) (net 11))
 (segment (start 122.174 100.076) (end 122.174 99.6315) (width 0.3) (layer F.Cu) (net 11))
 (segment (start 122.174 100.076) (end 122.301 100.076) (width 0.3) (layer F.Cu) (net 11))
 (segment (start 122.174 100.076) (end 122.199 100.076) (width 0.3) (layer F.Cu) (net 11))
 (segment (start 122.199 100.076) (end 125.501 96.774) (width 0.3) (layer F.Cu) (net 11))
 (segment (start 125.501 96.774) (end 125.501 94.6912) (width 0.3) (layer F.Cu) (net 11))
 (segment (start 125.501 94.6912) (end 126.365 93.8276) (width 0.3) (layer B.Cu) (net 11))
 (segment (start 126.365 93.8276) (end 126.365 92.5322) (width 0.3) (layer B.Cu) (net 11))
 (segment (start 126.365 92.5322) (end 127.787 91.1098) (width 0.3) (layer B.Cu) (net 11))
 (segment (start 127.787 91.1098) (end 128.245 91.1098) (width 0.3) (layer B.Cu) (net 11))
 (via (at 125.501 94.6912) (size 1.2) (drill 0.3) (layers F.Cu B.Cu) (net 11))
 (via (at 128.245 91.1098) (size 1.2) (drill 0.3) (layers F.Cu B.Cu) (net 11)))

